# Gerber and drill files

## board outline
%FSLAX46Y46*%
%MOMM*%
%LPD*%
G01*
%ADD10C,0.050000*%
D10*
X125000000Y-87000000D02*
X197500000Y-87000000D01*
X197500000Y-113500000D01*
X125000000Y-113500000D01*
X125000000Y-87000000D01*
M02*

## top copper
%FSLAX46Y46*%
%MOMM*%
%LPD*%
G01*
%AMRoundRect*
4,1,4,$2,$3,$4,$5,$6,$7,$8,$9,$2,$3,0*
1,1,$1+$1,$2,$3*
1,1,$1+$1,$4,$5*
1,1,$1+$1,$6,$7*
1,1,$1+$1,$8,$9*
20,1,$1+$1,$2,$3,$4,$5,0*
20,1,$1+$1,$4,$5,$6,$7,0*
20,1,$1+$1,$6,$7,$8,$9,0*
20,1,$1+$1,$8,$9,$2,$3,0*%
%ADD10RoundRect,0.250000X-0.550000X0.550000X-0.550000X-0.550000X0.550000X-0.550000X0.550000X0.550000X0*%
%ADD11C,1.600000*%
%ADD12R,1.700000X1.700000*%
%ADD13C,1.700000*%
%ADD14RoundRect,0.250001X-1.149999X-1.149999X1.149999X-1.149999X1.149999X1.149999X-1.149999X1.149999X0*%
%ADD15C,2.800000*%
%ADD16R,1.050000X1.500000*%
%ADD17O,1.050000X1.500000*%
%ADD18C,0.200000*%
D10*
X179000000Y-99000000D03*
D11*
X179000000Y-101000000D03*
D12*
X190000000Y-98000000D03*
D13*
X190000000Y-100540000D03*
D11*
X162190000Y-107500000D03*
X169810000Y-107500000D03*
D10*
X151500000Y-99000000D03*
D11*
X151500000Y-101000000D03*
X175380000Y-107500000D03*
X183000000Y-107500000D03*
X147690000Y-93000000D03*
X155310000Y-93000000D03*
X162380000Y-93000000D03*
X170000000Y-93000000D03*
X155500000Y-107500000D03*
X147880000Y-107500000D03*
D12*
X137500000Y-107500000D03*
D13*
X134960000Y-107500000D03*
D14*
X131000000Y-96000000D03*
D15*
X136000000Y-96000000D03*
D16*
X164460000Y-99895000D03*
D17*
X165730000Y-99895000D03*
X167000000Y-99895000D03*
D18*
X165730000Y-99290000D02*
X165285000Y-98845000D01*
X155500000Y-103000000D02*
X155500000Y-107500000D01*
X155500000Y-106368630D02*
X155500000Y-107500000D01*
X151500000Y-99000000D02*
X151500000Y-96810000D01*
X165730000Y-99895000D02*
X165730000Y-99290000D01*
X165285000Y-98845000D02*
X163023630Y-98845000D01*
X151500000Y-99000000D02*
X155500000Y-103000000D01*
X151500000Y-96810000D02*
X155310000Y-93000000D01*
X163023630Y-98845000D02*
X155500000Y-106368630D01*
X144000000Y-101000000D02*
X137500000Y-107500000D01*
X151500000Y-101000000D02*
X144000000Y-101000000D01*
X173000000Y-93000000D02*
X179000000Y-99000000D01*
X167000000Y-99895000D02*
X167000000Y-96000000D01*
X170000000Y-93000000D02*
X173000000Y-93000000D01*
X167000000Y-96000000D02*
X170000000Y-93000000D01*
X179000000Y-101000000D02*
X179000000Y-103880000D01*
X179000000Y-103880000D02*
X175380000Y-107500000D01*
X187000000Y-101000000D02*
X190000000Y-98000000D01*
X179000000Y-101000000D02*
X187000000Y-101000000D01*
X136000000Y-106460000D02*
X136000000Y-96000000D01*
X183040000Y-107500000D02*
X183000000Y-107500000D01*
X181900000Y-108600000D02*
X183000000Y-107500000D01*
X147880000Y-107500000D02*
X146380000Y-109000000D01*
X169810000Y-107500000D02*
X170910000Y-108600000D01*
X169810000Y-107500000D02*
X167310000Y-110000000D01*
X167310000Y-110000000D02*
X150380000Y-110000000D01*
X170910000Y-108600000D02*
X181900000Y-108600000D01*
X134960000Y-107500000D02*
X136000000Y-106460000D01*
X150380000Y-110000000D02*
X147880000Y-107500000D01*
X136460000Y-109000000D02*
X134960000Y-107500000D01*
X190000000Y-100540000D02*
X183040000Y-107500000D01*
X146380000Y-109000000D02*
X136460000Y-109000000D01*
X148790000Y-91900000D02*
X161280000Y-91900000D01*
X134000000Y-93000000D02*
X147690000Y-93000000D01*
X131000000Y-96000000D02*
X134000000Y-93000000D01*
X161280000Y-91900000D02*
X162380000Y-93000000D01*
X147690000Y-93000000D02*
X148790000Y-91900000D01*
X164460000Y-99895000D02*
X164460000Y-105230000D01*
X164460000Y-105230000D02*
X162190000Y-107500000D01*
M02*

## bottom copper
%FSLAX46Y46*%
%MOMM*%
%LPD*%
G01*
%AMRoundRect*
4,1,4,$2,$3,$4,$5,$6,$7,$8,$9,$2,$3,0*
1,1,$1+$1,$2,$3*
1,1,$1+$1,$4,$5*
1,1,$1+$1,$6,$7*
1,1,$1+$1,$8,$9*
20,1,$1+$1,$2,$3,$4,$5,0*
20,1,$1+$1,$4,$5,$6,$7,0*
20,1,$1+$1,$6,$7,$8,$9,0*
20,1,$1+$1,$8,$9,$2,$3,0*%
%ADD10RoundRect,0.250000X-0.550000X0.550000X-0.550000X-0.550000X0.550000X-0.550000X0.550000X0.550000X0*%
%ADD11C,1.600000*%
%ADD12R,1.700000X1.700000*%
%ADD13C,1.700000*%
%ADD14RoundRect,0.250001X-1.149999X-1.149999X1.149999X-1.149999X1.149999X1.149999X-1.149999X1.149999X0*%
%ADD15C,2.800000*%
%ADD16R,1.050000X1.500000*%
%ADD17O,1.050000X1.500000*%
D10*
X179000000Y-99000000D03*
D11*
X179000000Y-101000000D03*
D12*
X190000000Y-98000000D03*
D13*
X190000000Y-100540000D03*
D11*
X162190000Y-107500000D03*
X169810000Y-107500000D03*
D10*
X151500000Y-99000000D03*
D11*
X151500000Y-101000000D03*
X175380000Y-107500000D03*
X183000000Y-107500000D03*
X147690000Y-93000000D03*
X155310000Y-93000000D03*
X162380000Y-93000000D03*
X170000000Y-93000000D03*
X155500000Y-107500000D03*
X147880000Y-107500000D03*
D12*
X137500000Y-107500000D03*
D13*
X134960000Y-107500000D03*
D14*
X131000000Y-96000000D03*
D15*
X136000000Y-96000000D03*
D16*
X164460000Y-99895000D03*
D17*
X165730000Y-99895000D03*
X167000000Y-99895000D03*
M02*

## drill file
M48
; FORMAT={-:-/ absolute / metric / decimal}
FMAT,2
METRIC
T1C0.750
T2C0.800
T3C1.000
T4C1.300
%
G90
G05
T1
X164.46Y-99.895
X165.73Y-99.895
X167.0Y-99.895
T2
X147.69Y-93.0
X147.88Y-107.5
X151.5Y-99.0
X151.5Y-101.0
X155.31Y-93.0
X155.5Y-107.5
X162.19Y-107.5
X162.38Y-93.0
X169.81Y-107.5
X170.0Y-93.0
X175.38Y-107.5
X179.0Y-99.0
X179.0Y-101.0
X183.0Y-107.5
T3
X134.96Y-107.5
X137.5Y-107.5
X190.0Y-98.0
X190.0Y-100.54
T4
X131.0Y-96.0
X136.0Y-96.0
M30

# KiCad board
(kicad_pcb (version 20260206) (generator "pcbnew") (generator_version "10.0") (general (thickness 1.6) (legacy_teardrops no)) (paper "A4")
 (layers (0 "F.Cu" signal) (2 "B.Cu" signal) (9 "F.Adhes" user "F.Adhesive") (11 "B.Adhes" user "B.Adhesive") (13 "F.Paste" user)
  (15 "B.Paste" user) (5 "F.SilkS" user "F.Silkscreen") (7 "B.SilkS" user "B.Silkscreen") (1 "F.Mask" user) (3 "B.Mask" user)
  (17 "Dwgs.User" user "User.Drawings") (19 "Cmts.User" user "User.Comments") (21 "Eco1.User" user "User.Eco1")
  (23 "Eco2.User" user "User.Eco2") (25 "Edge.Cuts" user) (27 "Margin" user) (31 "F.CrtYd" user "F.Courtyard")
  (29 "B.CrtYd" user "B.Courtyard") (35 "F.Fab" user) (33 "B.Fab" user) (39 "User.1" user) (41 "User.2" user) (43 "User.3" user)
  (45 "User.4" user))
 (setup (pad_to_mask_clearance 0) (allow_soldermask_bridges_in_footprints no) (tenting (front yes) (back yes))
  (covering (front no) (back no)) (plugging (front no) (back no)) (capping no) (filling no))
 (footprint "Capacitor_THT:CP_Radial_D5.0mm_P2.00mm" (layer "F.Cu") (at 179 99 -90)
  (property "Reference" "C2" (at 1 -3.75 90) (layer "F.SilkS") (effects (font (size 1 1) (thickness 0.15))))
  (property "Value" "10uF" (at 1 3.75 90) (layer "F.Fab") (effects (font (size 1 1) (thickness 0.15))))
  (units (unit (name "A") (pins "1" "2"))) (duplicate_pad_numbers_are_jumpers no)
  (pad "1" thru_hole roundrect (at 0 0 270) (size 1.6 1.6) (drill 0.8) (layers "*.Cu" "*.Mask") (remove_unused_layers no)
   (roundrect_rratio 0.15625) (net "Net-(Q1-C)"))
  (pad "2" thru_hole circle (at 2 0 270) (size 1.6 1.6) (drill 0.8) (layers "*.Cu" "*.Mask") (remove_unused_layers no)
   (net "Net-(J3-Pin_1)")))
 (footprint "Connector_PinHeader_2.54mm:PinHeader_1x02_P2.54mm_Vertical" (layer "F.Cu") (at 190 98)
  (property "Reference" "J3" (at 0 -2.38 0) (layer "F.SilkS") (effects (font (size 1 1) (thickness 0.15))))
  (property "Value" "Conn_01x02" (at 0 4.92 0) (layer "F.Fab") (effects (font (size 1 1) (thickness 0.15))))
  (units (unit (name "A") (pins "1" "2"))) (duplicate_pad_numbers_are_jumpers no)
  (pad "1" thru_hole rect (at 0 0) (size 1.7 1.7) (drill 1) (layers "*.Cu" "*.Mask") (remove_unused_layers no) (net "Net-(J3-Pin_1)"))
  (pad "2" thru_hole circle (at 0 2.54) (size 1.7 1.7) (drill 1) (layers "*.Cu" "*.Mask") (remove_unused_layers no) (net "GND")))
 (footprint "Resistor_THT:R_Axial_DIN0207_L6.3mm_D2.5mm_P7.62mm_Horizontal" (layer "F.Cu") (at 162.19 107.5)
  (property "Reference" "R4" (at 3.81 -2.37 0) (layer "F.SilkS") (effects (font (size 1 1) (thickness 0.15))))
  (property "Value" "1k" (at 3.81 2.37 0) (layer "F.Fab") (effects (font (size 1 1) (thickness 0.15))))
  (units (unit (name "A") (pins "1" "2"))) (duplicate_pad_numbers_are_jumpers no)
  (pad "1" thru_hole circle (at 0 0) (size 1.6 1.6) (drill 0.8) (layers "*.Cu" "*.Mask") (remove_unused_layers no) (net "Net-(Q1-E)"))
  (pad "2" thru_hole circle (at 7.62 0) (size 1.6 1.6) (drill 0.8) (layers "*.Cu" "*.Mask") (remove_unused_layers no) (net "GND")))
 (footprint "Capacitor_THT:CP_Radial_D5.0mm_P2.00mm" (layer "F.Cu") (at 151.5 99 -90)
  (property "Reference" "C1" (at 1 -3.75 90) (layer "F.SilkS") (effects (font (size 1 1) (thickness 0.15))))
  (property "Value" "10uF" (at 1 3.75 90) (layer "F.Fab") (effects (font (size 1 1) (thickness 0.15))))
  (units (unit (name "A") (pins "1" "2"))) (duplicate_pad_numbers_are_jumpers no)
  (pad "1" thru_hole roundrect (at 0 0 270) (size 1.6 1.6) (drill 0.8) (layers "*.Cu" "*.Mask") (remove_unused_layers no)
   (roundrect_rratio 0.15625) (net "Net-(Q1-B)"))
  (pad "2" thru_hole circle (at 2 0 270) (size 1.6 1.6) (drill 0.8) (layers "*.Cu" "*.Mask") (remove_unused_layers no)
   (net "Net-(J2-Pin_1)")))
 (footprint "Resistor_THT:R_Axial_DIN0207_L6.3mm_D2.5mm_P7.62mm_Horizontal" (layer "F.Cu") (at 175.38 107.5)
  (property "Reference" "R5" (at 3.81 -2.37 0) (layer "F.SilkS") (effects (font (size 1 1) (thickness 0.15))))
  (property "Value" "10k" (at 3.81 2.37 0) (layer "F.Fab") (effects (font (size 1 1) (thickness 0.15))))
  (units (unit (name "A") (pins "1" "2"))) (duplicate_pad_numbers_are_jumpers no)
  (pad "1" thru_hole circle (at 0 0) (size 1.6 1.6) (drill 0.8) (layers "*.Cu" "*.Mask") (remove_unused_layers no) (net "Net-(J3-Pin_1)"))
  (pad "2" thru_hole circle (at 7.62 0) (size 1.6 1.6) (drill 0.8) (layers "*.Cu" "*.Mask") (remove_unused_layers no) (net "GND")))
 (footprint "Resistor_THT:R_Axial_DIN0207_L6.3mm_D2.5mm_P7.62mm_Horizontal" (layer "F.Cu") (at 147.69 93)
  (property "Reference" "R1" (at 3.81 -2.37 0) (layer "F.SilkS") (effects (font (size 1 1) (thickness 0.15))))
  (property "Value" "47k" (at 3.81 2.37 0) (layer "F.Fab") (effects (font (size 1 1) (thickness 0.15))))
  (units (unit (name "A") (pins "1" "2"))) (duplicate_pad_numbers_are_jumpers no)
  (pad "1" thru_hole circle (at 0 0) (size 1.6 1.6) (drill 0.8) (layers "*.Cu" "*.Mask") (remove_unused_layers no) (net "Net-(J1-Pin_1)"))
  (pad "2" thru_hole circle (at 7.62 0) (size 1.6 1.6) (drill 0.8) (layers "*.Cu" "*.Mask") (remove_unused_layers no) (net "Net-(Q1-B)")))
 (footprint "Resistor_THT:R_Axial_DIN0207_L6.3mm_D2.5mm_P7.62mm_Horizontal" (layer "F.Cu") (at 162.38 93)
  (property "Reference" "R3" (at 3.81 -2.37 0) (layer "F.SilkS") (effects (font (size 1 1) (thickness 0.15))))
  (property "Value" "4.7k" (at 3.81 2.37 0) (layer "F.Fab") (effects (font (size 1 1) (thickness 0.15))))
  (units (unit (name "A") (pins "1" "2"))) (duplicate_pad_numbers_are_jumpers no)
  (pad "1" thru_hole circle (at 0 0) (size 1.6 1.6) (drill 0.8) (layers "*.Cu" "*.Mask") (remove_unused_layers no) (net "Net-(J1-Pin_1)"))
  (pad "2" thru_hole circle (at 7.62 0) (size 1.6 1.6) (drill 0.8) (layers "*.Cu" "*.Mask") (remove_unused_layers no) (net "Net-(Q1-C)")))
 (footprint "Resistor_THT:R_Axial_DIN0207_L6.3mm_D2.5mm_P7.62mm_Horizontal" (layer "F.Cu") (at 155.5 107.5 180)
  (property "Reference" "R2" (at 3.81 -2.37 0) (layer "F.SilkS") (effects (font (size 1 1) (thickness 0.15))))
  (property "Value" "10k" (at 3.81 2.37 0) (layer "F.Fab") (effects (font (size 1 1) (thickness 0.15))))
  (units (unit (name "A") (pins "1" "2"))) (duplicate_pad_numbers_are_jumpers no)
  (pad "1" thru_hole circle (at 0 0 180) (size 1.6 1.6) (drill 0.8) (layers "*.Cu" "*.Mask") (remove_unused_layers no) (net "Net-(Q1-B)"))
  (pad "2" thru_hole circle (at 7.62 0 180) (size 1.6 1.6) (drill 0.8) (layers "*.Cu" "*.Mask") (remove_unused_layers no) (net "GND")))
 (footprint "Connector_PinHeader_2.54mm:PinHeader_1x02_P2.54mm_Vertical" (layer "F.Cu") (at 137.5 107.5 -90)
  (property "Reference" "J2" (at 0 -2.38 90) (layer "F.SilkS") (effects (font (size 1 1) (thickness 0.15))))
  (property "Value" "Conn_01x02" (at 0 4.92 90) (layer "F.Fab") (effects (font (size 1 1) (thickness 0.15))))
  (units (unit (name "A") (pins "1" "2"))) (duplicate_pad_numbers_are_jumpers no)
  (pad "1" thru_hole rect (at 0 0 270) (size 1.7 1.7) (drill 1) (layers "*.Cu" "*.Mask") (remove_unused_layers no) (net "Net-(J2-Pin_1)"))
  (pad "2" thru_hole circle (at 0 2.54 270) (size 1.7 1.7) (drill 1) (layers "*.Cu" "*.Mask") (remove_unused_layers no) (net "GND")))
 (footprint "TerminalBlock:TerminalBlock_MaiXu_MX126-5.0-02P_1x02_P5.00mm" (layer "F.Cu") (at 131 96)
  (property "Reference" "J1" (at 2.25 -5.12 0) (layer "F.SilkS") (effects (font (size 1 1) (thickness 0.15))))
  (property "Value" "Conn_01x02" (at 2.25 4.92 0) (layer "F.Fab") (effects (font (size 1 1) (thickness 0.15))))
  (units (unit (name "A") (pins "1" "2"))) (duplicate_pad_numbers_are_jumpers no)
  (pad "1" thru_hole roundrect (at 0 0) (size 2.8 2.8) (drill 1.3) (layers "*.Cu" "*.Mask") (remove_unused_layers no)
   (roundrect_rratio 0.089286) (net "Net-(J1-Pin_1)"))
  (pad "2" thru_hole circle (at 5 0) (size 2.8 2.8) (drill 1.3) (layers "*.Cu" "*.Mask") (remove_unused_layers no) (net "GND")))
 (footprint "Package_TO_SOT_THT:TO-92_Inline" (layer "F.Cu") (at 164.46 99.895)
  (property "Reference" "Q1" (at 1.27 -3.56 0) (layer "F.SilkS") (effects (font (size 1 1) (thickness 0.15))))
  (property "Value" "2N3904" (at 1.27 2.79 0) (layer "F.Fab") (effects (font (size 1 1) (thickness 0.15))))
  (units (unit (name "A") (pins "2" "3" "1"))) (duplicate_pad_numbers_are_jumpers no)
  (pad "1" thru_hole rect (at 0 0) (size 1.05 1.5) (drill 0.75) (layers "*.Cu" "*.Mask") (remove_unused_layers no) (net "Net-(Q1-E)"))
  (pad "2" thru_hole oval (at 1.27 0) (size 1.05 1.5) (drill 0.75) (layers "*.Cu" "*.Mask") (remove_unused_layers no) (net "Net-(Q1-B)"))
  (pad "3" thru_hole oval (at 2.54 0) (size 1.05 1.5) (drill 0.75) (layers "*.Cu" "*.Mask") (remove_unused_layers no) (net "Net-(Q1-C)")))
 (gr_rect (start 125 87) (end 197.5 113.5) (stroke (width 0.05) (type default)) (fill no) (layer "Edge.Cuts"))
 (segment (start 165.73 99.29) (end 165.285 98.845) (width 0.2) (layer "F.Cu") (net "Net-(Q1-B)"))
 (segment (start 155.5 103) (end 155.5 107.5) (width 0.2) (layer "F.Cu") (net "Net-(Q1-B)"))
 (segment (start 155.5 106.36863) (end 155.5 107.5) (width 0.2) (layer "F.Cu") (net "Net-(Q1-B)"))
 (segment (start 151.5 99) (end 151.5 96.81) (width 0.2) (layer "F.Cu") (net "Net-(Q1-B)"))
 (segment (start 165.73 99.895) (end 165.73 99.29) (width 0.2) (layer "F.Cu") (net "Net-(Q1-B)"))
 (segment (start 165.285 98.845) (end 163.02363 98.845) (width 0.2) (layer "F.Cu") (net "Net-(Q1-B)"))
 (segment (start 151.5 99) (end 155.5 103) (width 0.2) (layer "F.Cu") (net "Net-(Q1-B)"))
 (segment (start 151.5 96.81) (end 155.31 93) (width 0.2) (layer "F.Cu") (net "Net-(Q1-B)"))
 (segment (start 163.02363 98.845) (end 155.5 106.36863) (width 0.2) (layer "F.Cu") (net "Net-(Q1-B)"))
 (segment (start 144 101) (end 137.5 107.5) (width 0.2) (layer "F.Cu") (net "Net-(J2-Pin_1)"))
 (segment (start 151.5 101) (end 144 101) (width 0.2) (layer "F.Cu") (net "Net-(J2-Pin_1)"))
 (segment (start 173 93) (end 179 99) (width 0.2) (layer "F.Cu") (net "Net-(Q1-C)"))
 (segment (start 167 99.895) (end 167 96) (width 0.2) (layer "F.Cu") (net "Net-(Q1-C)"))
 (segment (start 170 93) (end 173 93) (width 0.2) (layer "F.Cu") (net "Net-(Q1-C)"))
 (segment (start 167 96) (end 170 93) (width 0.2) (layer "F.Cu") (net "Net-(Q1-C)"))
 (segment (start 179 101) (end 179 103.88) (width 0.2) (layer "F.Cu") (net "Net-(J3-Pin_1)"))
 (segment (start 179 103.88) (end 175.38 107.5) (width 0.2) (layer "F.Cu") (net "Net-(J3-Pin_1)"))
 (segment (start 187 101) (end 190 98) (width 0.2) (layer "F.Cu") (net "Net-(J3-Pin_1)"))
 (segment (start 179 101) (end 187 101) (width 0.2) (layer "F.Cu") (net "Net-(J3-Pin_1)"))
 (segment (start 136 106.46) (end 136 96) (width 0.2) (layer "F.Cu") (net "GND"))
 (segment (start 183.04 107.5) (end 183 107.5) (width 0.2) (layer "F.Cu") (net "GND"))
 (segment (start 181.9 108.6) (end 183 107.5) (width 0.2) (layer "F.Cu") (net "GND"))
 (segment (start 147.88 107.5) (end 146.38 109) (width 0.2) (layer "F.Cu") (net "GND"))
 (segment (start 169.81 107.5) (end 170.91 108.6) (width 0.2) (layer "F.Cu") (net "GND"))
 (segment (start 169.81 107.5) (end 167.31 110) (width 0.2) (layer "F.Cu") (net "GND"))
 (segment (start 167.31 110) (end 150.38 110) (width 0.2) (layer "F.Cu") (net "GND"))
 (segment (start 170.91 108.6) (end 181.9 108.6) (width 0.2) (layer "F.Cu") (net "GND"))
 (segment (start 134.96 107.5) (end 136 106.46) (width 0.2) (layer "F.Cu") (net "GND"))
 (segment (start 150.38 110) (end 147.88 107.5) (width 0.2) (layer "F.Cu") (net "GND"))
 (segment (start 136.46 109) (end 134.96 107.5) (width 0.2) (layer "F.Cu") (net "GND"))
 (segment (start 190 100.54) (end 183.04 107.5) (width 0.2) (layer "F.Cu") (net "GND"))
 (segment (start 146.38 109) (end 136.46 109) (width 0.2) (layer "F.Cu") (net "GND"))
 (segment (start 148.79 91.9) (end 161.28 91.9) (width 0.2) (layer "F.Cu") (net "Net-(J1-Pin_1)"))
 (segment (start 134 93) (end 147.69 93) (width 0.2) (layer "F.Cu") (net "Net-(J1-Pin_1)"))
 (segment (start 131 96) (end 134 93) (width 0.2) (layer "F.Cu") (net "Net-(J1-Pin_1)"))
 (segment (start 161.28 91.9) (end 162.38 93) (width 0.2) (layer "F.Cu") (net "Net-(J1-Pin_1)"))
 (segment (start 147.69 93) (end 148.79 91.9) (width 0.2) (layer "F.Cu") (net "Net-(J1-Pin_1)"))
 (segment (start 164.46 99.895) (end 164.46 105.23) (width 0.2) (layer "F.Cu") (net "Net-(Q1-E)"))
 (segment (start 164.46 105.23) (end 162.19 107.5) (width 0.2) (layer "F.Cu") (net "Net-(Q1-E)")))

